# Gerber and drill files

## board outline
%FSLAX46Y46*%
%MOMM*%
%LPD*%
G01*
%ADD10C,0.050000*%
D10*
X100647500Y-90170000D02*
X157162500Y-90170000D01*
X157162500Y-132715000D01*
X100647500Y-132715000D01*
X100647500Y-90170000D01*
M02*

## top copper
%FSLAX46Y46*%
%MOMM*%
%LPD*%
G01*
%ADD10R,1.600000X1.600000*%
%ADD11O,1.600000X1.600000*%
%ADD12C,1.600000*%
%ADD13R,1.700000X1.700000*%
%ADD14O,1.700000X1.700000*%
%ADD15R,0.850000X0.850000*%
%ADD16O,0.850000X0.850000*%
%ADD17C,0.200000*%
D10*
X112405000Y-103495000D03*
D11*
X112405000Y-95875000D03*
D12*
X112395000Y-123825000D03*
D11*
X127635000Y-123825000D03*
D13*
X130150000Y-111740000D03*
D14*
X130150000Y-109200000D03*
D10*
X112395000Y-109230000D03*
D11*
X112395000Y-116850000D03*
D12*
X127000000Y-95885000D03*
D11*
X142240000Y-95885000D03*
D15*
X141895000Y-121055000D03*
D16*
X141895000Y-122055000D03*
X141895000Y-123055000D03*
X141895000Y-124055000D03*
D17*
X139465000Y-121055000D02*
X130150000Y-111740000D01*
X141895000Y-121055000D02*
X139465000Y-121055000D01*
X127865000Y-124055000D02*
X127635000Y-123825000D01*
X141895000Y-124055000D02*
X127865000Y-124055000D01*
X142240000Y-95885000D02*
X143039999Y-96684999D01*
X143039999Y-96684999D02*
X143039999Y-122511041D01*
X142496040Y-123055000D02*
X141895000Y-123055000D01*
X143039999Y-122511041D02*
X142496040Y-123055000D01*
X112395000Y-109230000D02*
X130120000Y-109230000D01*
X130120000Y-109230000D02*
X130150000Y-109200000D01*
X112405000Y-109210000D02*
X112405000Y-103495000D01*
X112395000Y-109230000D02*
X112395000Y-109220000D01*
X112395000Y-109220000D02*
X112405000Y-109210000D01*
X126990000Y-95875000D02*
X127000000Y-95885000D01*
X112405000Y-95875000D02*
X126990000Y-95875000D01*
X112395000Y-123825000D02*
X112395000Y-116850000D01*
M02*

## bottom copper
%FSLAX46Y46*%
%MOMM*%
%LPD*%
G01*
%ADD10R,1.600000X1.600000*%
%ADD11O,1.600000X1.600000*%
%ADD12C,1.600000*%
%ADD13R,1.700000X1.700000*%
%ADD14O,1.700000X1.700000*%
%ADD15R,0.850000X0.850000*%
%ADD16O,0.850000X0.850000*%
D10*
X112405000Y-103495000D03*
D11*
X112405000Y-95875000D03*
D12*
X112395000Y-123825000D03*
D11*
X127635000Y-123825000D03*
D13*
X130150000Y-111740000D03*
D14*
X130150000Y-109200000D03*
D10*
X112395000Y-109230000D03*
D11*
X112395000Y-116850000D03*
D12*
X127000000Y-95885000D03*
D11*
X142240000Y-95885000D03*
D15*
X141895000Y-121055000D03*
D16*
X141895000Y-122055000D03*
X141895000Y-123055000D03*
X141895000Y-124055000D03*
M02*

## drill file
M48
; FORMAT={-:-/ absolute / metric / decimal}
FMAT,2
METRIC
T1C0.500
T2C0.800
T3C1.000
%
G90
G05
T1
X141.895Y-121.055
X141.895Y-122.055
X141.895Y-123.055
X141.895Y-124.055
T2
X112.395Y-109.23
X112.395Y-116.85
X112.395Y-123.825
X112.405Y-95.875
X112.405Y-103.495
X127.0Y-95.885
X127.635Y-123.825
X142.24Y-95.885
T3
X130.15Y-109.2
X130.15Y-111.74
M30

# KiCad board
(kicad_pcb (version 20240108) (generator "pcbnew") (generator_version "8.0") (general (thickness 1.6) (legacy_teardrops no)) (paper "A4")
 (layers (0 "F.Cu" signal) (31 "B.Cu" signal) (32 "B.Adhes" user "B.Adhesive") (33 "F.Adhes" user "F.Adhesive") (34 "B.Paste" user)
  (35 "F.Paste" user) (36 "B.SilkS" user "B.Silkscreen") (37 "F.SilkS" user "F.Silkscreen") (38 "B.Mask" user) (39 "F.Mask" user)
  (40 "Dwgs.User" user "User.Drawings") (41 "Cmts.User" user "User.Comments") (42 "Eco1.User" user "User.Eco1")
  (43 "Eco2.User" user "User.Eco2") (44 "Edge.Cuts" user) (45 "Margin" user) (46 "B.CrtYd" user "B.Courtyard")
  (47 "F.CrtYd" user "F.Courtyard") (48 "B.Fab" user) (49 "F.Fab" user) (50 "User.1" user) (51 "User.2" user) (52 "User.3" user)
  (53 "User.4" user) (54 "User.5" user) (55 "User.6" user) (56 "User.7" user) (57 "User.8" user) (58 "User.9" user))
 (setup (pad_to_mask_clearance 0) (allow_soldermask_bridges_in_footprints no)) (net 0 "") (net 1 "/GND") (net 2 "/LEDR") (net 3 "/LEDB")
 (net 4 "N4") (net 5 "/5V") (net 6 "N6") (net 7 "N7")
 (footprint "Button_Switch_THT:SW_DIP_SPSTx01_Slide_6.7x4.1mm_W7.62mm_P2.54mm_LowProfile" (layer "F.Cu") (at 112.405 103.495 90)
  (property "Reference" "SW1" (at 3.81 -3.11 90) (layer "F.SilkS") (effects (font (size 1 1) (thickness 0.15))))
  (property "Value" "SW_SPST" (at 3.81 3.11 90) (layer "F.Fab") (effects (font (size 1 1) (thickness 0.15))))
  (pad "1" thru_hole rect (at 0 0 90) (size 1.6 1.6) (drill 0.8) (layers "*.Cu" "*.Mask") (remove_unused_layers no) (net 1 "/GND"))
  (pad "2" thru_hole oval (at 7.62 0 90) (size 1.6 1.6) (drill 0.8) (layers "*.Cu" "*.Mask") (remove_unused_layers no) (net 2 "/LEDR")))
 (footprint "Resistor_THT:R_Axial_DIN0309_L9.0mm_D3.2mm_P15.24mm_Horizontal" (layer "F.Cu") (at 112.395 123.825)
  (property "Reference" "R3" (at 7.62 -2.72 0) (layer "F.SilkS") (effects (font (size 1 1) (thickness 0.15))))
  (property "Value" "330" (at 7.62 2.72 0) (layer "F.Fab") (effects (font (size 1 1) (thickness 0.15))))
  (pad "1" thru_hole circle (at 0 0) (size 1.6 1.6) (drill 0.8) (layers "*.Cu" "*.Mask") (remove_unused_layers no) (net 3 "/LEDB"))
  (pad "2" thru_hole oval (at 15.24 0) (size 1.6 1.6) (drill 0.8) (layers "*.Cu" "*.Mask") (remove_unused_layers no) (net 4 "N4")))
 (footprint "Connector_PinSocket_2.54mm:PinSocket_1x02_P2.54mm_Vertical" (layer "F.Cu") (at 130.15 111.74 180)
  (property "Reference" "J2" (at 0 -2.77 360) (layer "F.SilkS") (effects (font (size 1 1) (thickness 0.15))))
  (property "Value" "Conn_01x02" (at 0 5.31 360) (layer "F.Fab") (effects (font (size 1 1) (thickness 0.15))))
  (pad "1" thru_hole rect (at 0 0 180) (size 1.7 1.7) (drill 1) (layers "*.Cu" "*.Mask") (remove_unused_layers no) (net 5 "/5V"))
  (pad "2" thru_hole oval (at 0 2.54 180) (size 1.7 1.7) (drill 1) (layers "*.Cu" "*.Mask") (remove_unused_layers no) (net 1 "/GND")))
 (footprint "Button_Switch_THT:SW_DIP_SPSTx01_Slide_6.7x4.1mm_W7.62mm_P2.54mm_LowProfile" (layer "F.Cu") (at 112.395 109.23 -90)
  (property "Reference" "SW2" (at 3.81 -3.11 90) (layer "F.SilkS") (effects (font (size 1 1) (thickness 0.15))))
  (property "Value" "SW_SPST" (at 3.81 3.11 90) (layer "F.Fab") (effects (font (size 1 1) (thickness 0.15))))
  (pad "1" thru_hole rect (at 0 0 270) (size 1.6 1.6) (drill 0.8) (layers "*.Cu" "*.Mask") (remove_unused_layers no) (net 1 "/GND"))
  (pad "2" thru_hole oval (at 7.62 0 270) (size 1.6 1.6) (drill 0.8) (layers "*.Cu" "*.Mask") (remove_unused_layers no) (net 3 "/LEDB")))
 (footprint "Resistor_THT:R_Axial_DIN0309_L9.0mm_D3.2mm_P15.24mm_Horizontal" (layer "F.Cu") (at 127 95.885)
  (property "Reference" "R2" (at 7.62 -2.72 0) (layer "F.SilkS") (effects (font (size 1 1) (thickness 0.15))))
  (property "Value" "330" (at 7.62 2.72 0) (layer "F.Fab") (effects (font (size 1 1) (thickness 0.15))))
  (pad "1" thru_hole circle (at 0 0) (size 1.6 1.6) (drill 0.8) (layers "*.Cu" "*.Mask") (remove_unused_layers no) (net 2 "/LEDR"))
  (pad "2" thru_hole oval (at 15.24 0) (size 1.6 1.6) (drill 0.8) (layers "*.Cu" "*.Mask") (remove_unused_layers no) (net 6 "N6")))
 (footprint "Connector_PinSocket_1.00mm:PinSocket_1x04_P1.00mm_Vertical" (layer "F.Cu") (at 141.895 121.055)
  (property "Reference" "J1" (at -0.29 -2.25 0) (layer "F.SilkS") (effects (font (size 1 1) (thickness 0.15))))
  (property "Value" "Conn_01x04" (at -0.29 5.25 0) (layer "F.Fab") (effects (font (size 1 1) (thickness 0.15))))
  (pad "1" thru_hole rect (at 0 0) (size 0.85 0.85) (drill 0.5) (layers "*.Cu" "*.Mask") (remove_unused_layers no) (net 5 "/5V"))
  (pad "2" thru_hole oval (at 0 1) (size 0.85 0.85) (drill 0.5) (layers "*.Cu" "*.Mask") (remove_unused_layers no) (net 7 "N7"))
  (pad "3" thru_hole oval (at 0 2) (size 0.85 0.85) (drill 0.5) (layers "*.Cu" "*.Mask") (remove_unused_layers no) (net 6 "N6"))
  (pad "4" thru_hole oval (at 0 3) (size 0.85 0.85) (drill 0.5) (layers "*.Cu" "*.Mask") (remove_unused_layers no) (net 4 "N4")))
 (gr_rect (start 100.6475 90.17) (end 157.1625 132.715) (stroke (width 0.05) (type default)) (fill none) (layer "Edge.Cuts"))
 (segment (start 139.465 121.055) (end 130.15 111.74) (width 0.2) (layer "F.Cu") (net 5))
 (segment (start 141.895 121.055) (end 139.465 121.055) (width 0.2) (layer "F.Cu") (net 5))
 (segment (start 127.865 124.055) (end 127.635 123.825) (width 0.2) (layer "F.Cu") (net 4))
 (segment (start 141.895 124.055) (end 127.865 124.055) (width 0.2) (layer "F.Cu") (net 4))
 (segment (start 142.24 95.885) (end 143.039999 96.684999) (width 0.2) (layer "F.Cu") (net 6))
 (segment (start 143.039999 96.684999) (end 143.039999 122.511041) (width 0.2) (layer "F.Cu") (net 6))
 (segment (start 142.49604 123.055) (end 141.895 123.055) (width 0.2) (layer "F.Cu") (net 6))
 (segment (start 143.039999 122.511041) (end 142.49604 123.055) (width 0.2) (layer "F.Cu") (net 6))
 (segment (start 112.395 109.23) (end 130.12 109.23) (width 0.2) (layer "F.Cu") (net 1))
 (segment (start 130.12 109.23) (end 130.15 109.2) (width 0.2) (layer "F.Cu") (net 1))
 (segment (start 112.405 109.21) (end 112.405 103.495) (width 0.2) (layer "F.Cu") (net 1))
 (segment (start 112.395 109.23) (end 112.395 109.22) (width 0.2) (layer "F.Cu") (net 1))
 (segment (start 112.395 109.22) (end 112.405 109.21) (width 0.2) (layer "F.Cu") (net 1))
 (segment (start 126.99 95.875) (end 127 95.885) (width 0.2) (layer "F.Cu") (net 2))
 (segment (start 112.405 95.875) (end 126.99 95.875) (width 0.2) (layer "F.Cu") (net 2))
 (segment (start 112.395 123.825) (end 112.395 116.85) (width 0.2) (layer "F.Cu") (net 3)))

